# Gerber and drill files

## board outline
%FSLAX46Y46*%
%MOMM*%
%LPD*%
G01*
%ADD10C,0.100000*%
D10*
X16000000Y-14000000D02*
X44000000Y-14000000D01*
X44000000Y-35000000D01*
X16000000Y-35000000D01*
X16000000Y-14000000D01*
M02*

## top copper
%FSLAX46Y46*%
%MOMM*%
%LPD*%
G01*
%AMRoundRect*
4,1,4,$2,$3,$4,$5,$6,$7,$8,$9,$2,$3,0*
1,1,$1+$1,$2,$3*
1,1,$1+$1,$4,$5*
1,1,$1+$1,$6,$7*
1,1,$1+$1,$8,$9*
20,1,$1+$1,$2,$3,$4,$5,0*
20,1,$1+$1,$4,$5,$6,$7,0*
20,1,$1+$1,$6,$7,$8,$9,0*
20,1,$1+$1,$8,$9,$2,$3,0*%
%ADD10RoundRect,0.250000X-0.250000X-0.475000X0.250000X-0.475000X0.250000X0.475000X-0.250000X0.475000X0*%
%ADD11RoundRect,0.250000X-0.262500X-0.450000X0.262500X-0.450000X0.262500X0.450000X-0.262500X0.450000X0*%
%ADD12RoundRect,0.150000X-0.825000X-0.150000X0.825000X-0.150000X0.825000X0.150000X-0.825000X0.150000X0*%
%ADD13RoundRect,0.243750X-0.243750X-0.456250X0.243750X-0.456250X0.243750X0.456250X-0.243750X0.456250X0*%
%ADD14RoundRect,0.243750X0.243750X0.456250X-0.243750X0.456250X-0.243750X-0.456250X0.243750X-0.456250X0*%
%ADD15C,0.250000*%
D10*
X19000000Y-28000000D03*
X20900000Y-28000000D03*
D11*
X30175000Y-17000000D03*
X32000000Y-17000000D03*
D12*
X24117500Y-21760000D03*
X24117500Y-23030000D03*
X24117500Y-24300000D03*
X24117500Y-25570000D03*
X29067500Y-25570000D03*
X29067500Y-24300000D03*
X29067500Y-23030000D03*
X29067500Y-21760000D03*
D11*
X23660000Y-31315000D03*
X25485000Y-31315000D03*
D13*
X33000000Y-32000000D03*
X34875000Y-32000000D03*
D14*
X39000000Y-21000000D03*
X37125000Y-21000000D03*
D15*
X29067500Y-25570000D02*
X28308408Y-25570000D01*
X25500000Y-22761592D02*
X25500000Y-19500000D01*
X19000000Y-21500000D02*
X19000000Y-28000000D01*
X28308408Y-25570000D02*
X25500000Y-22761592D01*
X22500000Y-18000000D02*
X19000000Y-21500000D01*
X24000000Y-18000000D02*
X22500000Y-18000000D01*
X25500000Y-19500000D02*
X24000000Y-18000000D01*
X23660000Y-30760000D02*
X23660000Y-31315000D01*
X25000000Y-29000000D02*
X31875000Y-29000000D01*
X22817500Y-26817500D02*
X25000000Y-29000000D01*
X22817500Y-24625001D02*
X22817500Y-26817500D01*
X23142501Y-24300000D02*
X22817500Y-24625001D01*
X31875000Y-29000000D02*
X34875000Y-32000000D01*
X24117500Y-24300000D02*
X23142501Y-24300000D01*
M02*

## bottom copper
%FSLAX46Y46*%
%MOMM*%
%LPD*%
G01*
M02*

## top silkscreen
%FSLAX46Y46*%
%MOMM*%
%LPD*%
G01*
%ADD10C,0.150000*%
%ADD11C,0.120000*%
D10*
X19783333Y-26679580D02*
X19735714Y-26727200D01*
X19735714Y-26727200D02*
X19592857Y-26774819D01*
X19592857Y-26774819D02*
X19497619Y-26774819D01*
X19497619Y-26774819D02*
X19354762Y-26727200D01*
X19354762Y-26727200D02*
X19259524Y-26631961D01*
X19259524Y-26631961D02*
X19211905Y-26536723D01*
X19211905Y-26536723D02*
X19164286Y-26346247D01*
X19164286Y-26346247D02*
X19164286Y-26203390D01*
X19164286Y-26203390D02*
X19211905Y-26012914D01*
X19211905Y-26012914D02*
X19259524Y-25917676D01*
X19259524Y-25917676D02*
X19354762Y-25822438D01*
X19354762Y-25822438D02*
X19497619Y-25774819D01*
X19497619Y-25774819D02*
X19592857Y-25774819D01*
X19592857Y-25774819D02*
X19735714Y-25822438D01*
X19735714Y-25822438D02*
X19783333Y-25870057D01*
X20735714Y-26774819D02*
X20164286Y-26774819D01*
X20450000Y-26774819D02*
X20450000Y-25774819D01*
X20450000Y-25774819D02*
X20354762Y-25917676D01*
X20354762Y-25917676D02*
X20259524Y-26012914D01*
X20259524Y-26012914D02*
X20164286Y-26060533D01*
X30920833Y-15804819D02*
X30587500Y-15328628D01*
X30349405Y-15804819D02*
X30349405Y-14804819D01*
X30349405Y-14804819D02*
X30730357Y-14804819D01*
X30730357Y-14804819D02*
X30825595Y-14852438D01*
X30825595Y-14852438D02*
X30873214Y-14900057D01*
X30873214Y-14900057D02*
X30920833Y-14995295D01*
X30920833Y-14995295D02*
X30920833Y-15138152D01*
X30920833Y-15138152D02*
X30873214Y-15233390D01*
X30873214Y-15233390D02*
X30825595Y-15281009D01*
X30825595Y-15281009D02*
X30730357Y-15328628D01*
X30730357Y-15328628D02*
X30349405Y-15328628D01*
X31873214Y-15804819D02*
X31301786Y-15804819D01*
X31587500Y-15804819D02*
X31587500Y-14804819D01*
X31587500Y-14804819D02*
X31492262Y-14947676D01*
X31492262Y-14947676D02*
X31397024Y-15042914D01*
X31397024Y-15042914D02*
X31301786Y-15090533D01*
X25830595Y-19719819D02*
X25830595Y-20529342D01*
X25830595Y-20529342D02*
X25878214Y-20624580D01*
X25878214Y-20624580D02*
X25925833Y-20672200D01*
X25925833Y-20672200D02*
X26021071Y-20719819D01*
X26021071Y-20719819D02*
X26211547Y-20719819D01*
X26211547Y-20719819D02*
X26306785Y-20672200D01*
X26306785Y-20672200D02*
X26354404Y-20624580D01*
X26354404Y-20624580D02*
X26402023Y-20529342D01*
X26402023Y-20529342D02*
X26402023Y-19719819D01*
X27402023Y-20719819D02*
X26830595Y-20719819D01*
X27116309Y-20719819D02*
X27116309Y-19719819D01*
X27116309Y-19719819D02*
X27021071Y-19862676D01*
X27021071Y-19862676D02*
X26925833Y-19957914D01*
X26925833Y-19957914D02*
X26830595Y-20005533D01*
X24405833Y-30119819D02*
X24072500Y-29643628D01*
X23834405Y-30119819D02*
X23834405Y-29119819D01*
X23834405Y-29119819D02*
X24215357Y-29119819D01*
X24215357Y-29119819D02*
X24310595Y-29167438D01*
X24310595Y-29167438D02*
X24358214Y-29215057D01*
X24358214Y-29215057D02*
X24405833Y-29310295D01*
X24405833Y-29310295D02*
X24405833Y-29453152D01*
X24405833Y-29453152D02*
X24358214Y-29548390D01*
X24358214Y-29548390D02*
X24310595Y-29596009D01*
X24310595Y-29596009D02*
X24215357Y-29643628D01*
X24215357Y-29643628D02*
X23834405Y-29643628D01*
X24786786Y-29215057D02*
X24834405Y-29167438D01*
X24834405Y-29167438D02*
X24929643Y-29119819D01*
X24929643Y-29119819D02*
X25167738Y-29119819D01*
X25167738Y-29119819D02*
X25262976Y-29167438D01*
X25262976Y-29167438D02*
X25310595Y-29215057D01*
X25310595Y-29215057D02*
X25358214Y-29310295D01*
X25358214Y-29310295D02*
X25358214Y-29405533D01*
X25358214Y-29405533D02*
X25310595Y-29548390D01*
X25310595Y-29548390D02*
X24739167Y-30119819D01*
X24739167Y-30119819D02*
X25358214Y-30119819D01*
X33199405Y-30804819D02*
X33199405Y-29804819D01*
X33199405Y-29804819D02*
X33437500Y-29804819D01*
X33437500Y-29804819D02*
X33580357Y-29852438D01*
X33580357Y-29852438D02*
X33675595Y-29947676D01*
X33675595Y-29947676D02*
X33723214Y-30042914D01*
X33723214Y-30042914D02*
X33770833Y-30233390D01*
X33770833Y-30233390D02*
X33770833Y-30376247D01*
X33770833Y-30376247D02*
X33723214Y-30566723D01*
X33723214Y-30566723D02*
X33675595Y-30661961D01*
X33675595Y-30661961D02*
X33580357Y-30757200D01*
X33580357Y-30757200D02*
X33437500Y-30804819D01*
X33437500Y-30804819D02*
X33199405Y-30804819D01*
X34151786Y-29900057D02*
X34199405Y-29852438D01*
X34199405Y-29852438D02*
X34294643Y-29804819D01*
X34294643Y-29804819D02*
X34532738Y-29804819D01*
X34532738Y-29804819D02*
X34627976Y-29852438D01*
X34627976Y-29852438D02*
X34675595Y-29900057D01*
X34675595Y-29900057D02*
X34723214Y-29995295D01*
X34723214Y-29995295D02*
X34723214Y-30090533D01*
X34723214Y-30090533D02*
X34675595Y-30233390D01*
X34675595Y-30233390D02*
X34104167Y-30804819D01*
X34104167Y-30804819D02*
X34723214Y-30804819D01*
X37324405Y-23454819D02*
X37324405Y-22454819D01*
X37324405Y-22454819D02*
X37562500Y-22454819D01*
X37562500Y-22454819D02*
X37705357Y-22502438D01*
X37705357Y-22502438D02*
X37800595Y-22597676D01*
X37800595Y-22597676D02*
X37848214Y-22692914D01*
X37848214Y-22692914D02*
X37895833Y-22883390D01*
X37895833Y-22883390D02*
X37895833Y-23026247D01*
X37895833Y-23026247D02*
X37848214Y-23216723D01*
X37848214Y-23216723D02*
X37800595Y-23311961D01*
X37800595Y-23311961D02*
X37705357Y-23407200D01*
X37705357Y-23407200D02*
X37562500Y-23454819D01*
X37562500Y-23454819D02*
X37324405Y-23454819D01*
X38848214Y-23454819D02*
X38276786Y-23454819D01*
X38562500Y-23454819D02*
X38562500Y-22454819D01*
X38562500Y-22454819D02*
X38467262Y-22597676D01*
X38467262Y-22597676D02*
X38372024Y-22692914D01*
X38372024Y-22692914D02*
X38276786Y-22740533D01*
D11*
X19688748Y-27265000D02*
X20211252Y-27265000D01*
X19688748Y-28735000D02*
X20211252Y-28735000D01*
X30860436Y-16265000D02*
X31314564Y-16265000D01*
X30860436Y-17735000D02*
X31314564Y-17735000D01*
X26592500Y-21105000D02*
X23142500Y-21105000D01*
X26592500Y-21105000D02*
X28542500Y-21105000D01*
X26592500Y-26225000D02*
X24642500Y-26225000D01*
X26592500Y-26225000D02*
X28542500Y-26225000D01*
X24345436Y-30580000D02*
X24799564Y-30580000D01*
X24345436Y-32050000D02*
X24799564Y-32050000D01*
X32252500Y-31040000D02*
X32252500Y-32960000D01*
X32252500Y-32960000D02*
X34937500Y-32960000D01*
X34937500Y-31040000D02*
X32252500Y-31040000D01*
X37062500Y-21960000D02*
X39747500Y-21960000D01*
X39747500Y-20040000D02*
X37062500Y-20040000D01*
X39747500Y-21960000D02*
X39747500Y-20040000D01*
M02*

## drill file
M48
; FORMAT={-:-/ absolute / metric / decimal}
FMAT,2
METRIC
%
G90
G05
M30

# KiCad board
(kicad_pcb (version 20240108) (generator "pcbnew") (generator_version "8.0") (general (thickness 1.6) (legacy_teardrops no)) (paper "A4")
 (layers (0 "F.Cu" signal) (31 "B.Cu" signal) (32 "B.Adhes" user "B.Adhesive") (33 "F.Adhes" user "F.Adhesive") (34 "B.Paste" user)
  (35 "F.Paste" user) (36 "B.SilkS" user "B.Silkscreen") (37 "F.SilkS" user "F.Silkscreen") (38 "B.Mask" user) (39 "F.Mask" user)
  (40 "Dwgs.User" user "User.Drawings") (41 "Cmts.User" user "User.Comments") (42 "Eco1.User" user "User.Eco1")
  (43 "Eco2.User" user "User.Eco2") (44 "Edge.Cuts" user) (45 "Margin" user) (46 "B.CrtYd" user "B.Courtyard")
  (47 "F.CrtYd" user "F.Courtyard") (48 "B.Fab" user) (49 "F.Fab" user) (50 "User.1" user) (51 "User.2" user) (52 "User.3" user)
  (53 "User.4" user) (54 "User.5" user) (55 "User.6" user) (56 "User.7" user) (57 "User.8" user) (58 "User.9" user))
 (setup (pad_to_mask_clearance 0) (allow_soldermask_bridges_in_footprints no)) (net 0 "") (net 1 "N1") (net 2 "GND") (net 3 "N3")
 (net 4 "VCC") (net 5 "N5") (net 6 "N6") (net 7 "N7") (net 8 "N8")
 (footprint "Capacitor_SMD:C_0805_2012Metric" (layer "F.Cu") (at 19.95 28)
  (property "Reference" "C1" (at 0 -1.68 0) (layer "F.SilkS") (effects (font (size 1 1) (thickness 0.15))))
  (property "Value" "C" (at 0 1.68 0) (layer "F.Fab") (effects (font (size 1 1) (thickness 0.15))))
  (fp_line (start -0.261252 -0.735) (end 0.261252 -0.735) (stroke (width 0.12) (type solid)) (layer "F.SilkS"))
  (fp_line (start -0.261252 0.735) (end 0.261252 0.735) (stroke (width 0.12) (type solid)) (layer "F.SilkS"))
  (pad "1" smd roundrect (at -0.95 0) (size 1 1.45) (layers "F.Cu" "F.Paste" "F.Mask") (roundrect_rratio 0.25) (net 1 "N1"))
  (pad "2" smd roundrect (at 0.95 0) (size 1 1.45) (layers "F.Cu" "F.Paste" "F.Mask") (roundrect_rratio 0.25) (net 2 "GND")))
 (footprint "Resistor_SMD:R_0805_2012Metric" (layer "F.Cu") (at 31.0875 17)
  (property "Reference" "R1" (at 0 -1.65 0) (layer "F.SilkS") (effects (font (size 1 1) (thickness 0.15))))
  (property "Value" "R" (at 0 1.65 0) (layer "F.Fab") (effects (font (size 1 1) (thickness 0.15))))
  (fp_line (start -0.227064 -0.735) (end 0.227064 -0.735) (stroke (width 0.12) (type solid)) (layer "F.SilkS"))
  (fp_line (start -0.227064 0.735) (end 0.227064 0.735) (stroke (width 0.12) (type solid)) (layer "F.SilkS"))
  (pad "1" smd roundrect (at -0.9125 0) (size 1.025 1.4) (layers "F.Cu" "F.Paste" "F.Mask") (roundrect_rratio 0.243902) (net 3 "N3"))
  (pad "2" smd roundrect (at 0.9125 0) (size 1.025 1.4) (layers "F.Cu" "F.Paste" "F.Mask") (roundrect_rratio 0.243902) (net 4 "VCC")))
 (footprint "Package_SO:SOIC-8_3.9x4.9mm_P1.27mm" (layer "F.Cu") (at 26.5925 23.665)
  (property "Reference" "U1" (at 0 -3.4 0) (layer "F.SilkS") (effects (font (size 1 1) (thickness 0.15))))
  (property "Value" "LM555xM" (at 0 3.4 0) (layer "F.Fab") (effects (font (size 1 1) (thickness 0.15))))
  (fp_line (start 0 -2.56) (end -3.45 -2.56) (stroke (width 0.12) (type solid)) (layer "F.SilkS"))
  (fp_line (start 0 -2.56) (end 1.95 -2.56) (stroke (width 0.12) (type solid)) (layer "F.SilkS"))
  (fp_line (start 0 2.56) (end -1.95 2.56) (stroke (width 0.12) (type solid)) (layer "F.SilkS"))
  (fp_line (start 0 2.56) (end 1.95 2.56) (stroke (width 0.12) (type solid)) (layer "F.SilkS"))
  (pad "1" smd roundrect (at -2.475 -1.905) (size 1.95 0.6) (layers "F.Cu" "F.Paste" "F.Mask") (roundrect_rratio 0.25) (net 2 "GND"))
  (pad "2" smd roundrect (at -2.475 -0.635) (size 1.95 0.6) (layers "F.Cu" "F.Paste" "F.Mask") (roundrect_rratio 0.25) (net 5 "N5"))
  (pad "3" smd roundrect (at -2.475 0.635) (size 1.95 0.6) (layers "F.Cu" "F.Paste" "F.Mask") (roundrect_rratio 0.25) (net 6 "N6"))
  (pad "4" smd roundrect (at -2.475 1.905) (size 1.95 0.6) (layers "F.Cu" "F.Paste" "F.Mask") (roundrect_rratio 0.25) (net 4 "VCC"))
  (pad "5" smd roundrect (at 2.475 1.905) (size 1.95 0.6) (layers "F.Cu" "F.Paste" "F.Mask") (roundrect_rratio 0.25) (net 1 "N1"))
  (pad "6" smd roundrect (at 2.475 0.635) (size 1.95 0.6) (layers "F.Cu" "F.Paste" "F.Mask") (roundrect_rratio 0.25) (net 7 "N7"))
  (pad "7" smd roundrect (at 2.475 -0.635) (size 1.95 0.6) (layers "F.Cu" "F.Paste" "F.Mask") (roundrect_rratio 0.25) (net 7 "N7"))
  (pad "8" smd roundrect (at 2.475 -1.905) (size 1.95 0.6) (layers "F.Cu" "F.Paste" "F.Mask") (roundrect_rratio 0.25) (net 4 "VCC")))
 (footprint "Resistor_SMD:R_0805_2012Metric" (layer "F.Cu") (at 24.5725 31.315)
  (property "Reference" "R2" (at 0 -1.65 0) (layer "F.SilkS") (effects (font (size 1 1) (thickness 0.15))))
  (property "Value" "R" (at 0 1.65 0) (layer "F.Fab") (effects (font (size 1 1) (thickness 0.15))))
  (fp_line (start -0.227064 -0.735) (end 0.227064 -0.735) (stroke (width 0.12) (type solid)) (layer "F.SilkS"))
  (fp_line (start -0.227064 0.735) (end 0.227064 0.735) (stroke (width 0.12) (type solid)) (layer "F.SilkS"))
  (pad "1" smd roundrect (at -0.9125 0) (size 1.025 1.4) (layers "F.Cu" "F.Paste" "F.Mask") (roundrect_rratio 0.243902) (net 2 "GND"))
  (pad "2" smd roundrect (at 0.9125 0) (size 1.025 1.4) (layers "F.Cu" "F.Paste" "F.Mask") (roundrect_rratio 0.243902) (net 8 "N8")))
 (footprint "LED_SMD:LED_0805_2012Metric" (layer "F.Cu") (at 33.9375 32)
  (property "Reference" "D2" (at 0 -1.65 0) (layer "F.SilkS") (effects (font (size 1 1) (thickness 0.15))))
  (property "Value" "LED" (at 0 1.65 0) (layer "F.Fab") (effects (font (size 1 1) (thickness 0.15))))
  (fp_line (start -1.685 -0.96) (end -1.685 0.96) (stroke (width 0.12) (type solid)) (layer "F.SilkS"))
  (fp_line (start -1.685 0.96) (end 1 0.96) (stroke (width 0.12) (type solid)) (layer "F.SilkS"))
  (fp_line (start 1 -0.96) (end -1.685 -0.96) (stroke (width 0.12) (type solid)) (layer "F.SilkS"))
  (pad "1" smd roundrect (at -0.9375 0) (size 0.975 1.4) (layers "F.Cu" "F.Paste" "F.Mask") (roundrect_rratio 0.25) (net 8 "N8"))
  (pad "2" smd roundrect (at 0.9375 0) (size 0.975 1.4) (layers "F.Cu" "F.Paste" "F.Mask") (roundrect_rratio 0.25) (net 6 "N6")))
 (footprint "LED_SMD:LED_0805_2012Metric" (layer "F.Cu") (at 38.0625 21 180)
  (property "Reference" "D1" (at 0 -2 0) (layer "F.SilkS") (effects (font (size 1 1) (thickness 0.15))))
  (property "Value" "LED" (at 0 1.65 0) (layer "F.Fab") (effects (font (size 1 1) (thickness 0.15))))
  (fp_line (start 1 -0.96) (end -1.685 -0.96) (stroke (width 0.12) (type solid)) (layer "F.SilkS"))
  (fp_line (start -1.685 0.96) (end 1 0.96) (stroke (width 0.12) (type solid)) (layer "F.SilkS"))
  (fp_line (start -1.685 -0.96) (end -1.685 0.96) (stroke (width 0.12) (type solid)) (layer "F.SilkS"))
  (pad "1" smd roundrect (at -0.9375 0 180) (size 0.975 1.4) (layers "F.Cu" "F.Paste" "F.Mask") (roundrect_rratio 0.25) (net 6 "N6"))
  (pad "2" smd roundrect (at 0.9375 0 180) (size 0.975 1.4) (layers "F.Cu" "F.Paste" "F.Mask") (roundrect_rratio 0.25) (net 3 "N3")))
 (gr_rect (start 16 14) (end 44 35) (stroke (width 0.1) (type default)) (fill none) (layer "Edge.Cuts"))
 (segment (start 29.0675 25.57) (end 28.308408 25.57) (width 0.25) (layer "F.Cu") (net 1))
 (segment (start 25.5 22.761592) (end 25.5 19.5) (width 0.25) (layer "F.Cu") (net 1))
 (segment (start 19 21.5) (end 19 28) (width 0.25) (layer "F.Cu") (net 1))
 (segment (start 28.308408 25.57) (end 25.5 22.761592) (width 0.25) (layer "F.Cu") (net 1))
 (segment (start 22.5 18) (end 19 21.5) (width 0.25) (layer "F.Cu") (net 1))
 (segment (start 24 18) (end 22.5 18) (width 0.25) (layer "F.Cu") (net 1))
 (segment (start 25.5 19.5) (end 24 18) (width 0.25) (layer "F.Cu") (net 1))
 (segment (start 23.66 30.76) (end 23.66 31.315) (width 0.25) (layer "F.Cu") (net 2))
 (segment (start 25 29) (end 31.875 29) (width 0.25) (layer "F.Cu") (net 6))
 (segment (start 22.8175 26.8175) (end 25 29) (width 0.25) (layer "F.Cu") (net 6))
 (segment (start 22.8175 24.625001) (end 22.8175 26.8175) (width 0.25) (layer "F.Cu") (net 6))
 (segment (start 23.142501 24.3) (end 22.8175 24.625001) (width 0.25) (layer "F.Cu") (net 6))
 (segment (start 31.875 29) (end 34.875 32) (width 0.25) (layer "F.Cu") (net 6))
 (segment (start 24.1175 24.3) (end 23.142501 24.3) (width 0.25) (layer "F.Cu") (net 6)))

